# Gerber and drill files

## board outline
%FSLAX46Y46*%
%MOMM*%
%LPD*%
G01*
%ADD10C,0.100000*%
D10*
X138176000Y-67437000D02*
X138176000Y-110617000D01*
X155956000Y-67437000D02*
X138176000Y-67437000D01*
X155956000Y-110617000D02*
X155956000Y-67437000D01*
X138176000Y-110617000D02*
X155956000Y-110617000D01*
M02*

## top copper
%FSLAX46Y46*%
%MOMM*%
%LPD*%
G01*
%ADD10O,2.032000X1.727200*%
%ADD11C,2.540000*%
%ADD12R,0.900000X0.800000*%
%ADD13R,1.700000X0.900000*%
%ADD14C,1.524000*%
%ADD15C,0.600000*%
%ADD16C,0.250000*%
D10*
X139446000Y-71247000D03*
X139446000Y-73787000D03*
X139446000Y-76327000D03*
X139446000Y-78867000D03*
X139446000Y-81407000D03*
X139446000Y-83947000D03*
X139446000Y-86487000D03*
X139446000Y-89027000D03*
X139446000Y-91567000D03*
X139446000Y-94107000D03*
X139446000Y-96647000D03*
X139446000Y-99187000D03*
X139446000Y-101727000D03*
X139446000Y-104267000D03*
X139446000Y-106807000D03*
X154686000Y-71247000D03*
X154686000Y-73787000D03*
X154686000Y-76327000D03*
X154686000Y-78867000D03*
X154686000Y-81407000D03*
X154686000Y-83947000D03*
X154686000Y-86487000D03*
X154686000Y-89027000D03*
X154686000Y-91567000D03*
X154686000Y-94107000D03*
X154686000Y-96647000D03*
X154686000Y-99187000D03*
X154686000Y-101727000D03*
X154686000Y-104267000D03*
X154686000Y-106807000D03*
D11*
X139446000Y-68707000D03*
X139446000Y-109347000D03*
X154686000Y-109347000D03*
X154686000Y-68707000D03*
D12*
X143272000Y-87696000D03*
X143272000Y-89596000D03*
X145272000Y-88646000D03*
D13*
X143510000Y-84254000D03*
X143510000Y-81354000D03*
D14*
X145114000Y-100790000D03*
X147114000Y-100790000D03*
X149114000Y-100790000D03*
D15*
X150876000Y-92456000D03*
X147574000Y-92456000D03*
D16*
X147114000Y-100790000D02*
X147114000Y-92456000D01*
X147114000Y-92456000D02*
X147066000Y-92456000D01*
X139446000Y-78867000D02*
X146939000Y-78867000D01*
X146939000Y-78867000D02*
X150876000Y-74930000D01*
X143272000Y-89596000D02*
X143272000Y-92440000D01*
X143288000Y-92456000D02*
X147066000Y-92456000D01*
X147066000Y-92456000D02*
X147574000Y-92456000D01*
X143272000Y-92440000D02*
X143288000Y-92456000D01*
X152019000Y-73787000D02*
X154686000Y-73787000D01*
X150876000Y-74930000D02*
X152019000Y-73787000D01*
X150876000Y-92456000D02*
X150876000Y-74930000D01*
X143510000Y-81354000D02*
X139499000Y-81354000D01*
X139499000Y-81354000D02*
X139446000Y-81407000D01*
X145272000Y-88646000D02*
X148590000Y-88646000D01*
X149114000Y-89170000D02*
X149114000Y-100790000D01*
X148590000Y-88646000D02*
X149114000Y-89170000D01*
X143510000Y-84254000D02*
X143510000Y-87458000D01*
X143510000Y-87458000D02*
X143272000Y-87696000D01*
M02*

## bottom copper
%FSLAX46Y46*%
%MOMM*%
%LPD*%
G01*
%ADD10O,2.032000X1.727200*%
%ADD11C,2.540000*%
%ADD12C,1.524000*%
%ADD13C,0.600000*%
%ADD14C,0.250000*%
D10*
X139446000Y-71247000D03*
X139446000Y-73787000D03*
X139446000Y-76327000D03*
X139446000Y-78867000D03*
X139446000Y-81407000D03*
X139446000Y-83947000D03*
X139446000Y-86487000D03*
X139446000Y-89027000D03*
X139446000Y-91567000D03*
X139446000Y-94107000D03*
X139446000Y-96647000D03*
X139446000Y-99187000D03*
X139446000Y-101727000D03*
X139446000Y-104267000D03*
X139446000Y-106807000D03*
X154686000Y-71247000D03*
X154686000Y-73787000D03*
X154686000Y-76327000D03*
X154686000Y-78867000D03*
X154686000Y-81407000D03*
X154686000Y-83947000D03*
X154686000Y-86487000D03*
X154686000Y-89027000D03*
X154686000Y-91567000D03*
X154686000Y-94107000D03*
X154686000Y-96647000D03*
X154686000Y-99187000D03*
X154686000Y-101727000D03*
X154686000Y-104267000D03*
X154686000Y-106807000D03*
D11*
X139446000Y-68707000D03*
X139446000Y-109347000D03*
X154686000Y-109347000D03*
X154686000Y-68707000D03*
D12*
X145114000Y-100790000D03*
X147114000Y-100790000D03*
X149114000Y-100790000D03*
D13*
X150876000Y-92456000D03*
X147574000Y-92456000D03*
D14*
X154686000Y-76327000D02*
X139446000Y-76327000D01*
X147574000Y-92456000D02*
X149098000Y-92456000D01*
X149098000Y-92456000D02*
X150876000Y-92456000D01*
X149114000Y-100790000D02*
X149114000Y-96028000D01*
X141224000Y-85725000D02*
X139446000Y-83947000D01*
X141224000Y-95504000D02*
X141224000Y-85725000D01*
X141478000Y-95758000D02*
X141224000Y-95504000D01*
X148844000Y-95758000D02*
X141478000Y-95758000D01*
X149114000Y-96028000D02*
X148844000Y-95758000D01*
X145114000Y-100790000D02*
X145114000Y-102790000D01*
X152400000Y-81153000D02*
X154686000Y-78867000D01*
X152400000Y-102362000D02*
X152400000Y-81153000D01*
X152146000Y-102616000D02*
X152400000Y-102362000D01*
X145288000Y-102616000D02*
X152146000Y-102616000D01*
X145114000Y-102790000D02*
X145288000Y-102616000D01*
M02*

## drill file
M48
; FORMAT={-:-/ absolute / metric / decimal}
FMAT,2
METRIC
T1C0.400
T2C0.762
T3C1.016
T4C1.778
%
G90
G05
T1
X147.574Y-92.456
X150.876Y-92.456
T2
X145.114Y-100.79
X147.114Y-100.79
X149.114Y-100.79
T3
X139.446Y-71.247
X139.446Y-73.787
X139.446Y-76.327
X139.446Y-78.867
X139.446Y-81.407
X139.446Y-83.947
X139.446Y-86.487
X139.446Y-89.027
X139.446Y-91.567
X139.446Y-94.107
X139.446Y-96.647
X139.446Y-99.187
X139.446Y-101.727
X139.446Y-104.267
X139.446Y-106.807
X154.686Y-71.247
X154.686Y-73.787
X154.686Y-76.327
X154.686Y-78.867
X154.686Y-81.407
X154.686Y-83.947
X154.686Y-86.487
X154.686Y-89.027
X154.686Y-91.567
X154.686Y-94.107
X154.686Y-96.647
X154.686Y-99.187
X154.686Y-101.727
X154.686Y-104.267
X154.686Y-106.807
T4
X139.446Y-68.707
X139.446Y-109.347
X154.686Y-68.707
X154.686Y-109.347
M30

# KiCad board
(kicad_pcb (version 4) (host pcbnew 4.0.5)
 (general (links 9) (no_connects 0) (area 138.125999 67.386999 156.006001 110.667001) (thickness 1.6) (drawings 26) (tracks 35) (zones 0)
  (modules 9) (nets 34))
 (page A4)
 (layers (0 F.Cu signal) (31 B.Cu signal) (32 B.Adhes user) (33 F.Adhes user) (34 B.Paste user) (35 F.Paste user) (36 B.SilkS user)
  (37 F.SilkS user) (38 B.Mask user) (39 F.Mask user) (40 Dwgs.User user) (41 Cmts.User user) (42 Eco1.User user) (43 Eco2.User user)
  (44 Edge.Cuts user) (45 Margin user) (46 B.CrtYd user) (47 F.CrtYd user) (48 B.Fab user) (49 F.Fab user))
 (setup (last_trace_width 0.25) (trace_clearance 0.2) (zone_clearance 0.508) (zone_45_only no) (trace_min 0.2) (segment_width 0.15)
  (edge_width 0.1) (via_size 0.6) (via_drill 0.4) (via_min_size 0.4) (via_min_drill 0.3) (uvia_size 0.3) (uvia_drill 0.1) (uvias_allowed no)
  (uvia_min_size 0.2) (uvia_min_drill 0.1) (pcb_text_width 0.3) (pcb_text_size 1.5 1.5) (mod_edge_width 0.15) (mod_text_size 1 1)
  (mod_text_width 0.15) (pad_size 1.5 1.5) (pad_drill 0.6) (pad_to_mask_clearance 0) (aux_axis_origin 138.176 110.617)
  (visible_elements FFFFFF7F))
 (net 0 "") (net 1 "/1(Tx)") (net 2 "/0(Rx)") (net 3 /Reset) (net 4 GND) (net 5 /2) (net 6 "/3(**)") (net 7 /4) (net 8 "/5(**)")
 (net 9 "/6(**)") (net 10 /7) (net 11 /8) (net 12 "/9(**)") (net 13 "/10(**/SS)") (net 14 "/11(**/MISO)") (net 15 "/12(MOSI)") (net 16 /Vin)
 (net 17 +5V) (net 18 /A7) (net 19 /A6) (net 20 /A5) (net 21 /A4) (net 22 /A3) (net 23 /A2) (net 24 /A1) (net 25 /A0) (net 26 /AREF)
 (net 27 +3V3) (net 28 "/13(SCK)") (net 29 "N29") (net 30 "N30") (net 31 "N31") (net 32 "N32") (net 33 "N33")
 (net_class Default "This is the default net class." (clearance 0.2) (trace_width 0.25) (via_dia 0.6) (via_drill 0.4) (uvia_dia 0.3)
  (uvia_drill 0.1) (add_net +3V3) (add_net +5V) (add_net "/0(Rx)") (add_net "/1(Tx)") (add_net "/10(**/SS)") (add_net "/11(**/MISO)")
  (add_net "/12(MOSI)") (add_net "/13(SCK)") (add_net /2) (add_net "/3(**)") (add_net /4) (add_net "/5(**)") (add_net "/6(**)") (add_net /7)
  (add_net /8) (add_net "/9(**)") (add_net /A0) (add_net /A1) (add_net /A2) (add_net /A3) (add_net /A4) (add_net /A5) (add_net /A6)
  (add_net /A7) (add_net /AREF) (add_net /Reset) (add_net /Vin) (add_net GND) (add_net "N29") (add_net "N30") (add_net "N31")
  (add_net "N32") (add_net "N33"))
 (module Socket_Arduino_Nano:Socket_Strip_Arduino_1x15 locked (layer F.Cu) (at 139.446 71.247 270)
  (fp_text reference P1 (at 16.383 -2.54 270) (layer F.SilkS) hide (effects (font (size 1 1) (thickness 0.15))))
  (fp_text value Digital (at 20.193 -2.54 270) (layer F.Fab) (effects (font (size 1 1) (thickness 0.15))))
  (pad 1 thru_hole oval (at 0 0 270) (size 1.7272 2.032) (drill 1.016) (layers *.Cu *.Mask F.SilkS) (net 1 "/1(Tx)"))
  (pad 2 thru_hole oval (at 2.54 0 270) (size 1.7272 2.032) (drill 1.016) (layers *.Cu *.Mask F.SilkS) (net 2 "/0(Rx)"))
  (pad 3 thru_hole oval (at 5.08 0 270) (size 1.7272 2.032) (drill 1.016) (layers *.Cu *.Mask F.SilkS) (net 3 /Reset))
  (pad 4 thru_hole oval (at 7.62 0 270) (size 1.7272 2.032) (drill 1.016) (layers *.Cu *.Mask F.SilkS) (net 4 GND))
  (pad 5 thru_hole oval (at 10.16 0 270) (size 1.7272 2.032) (drill 1.016) (layers *.Cu *.Mask F.SilkS) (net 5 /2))
  (pad 6 thru_hole oval (at 12.7 0 270) (size 1.7272 2.032) (drill 1.016) (layers *.Cu *.Mask F.SilkS) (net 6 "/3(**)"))
  (pad 7 thru_hole oval (at 15.24 0 270) (size 1.7272 2.032) (drill 1.016) (layers *.Cu *.Mask F.SilkS) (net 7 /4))
  (pad 8 thru_hole oval (at 17.78 0 270) (size 1.7272 2.032) (drill 1.016) (layers *.Cu *.Mask F.SilkS) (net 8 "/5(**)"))
  (pad 9 thru_hole oval (at 20.32 0 270) (size 1.7272 2.032) (drill 1.016) (layers *.Cu *.Mask F.SilkS) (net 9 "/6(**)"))
  (pad 10 thru_hole oval (at 22.86 0 270) (size 1.7272 2.032) (drill 1.016) (layers *.Cu *.Mask F.SilkS) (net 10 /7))
  (pad 11 thru_hole oval (at 25.4 0 270) (size 1.7272 2.032) (drill 1.016) (layers *.Cu *.Mask F.SilkS) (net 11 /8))
  (pad 12 thru_hole oval (at 27.94 0 270) (size 1.7272 2.032) (drill 1.016) (layers *.Cu *.Mask F.SilkS) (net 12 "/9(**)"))
  (pad 13 thru_hole oval (at 30.48 0 270) (size 1.7272 2.032) (drill 1.016) (layers *.Cu *.Mask F.SilkS) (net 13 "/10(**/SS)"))
  (pad 14 thru_hole oval (at 33.02 0 270) (size 1.7272 2.032) (drill 1.016) (layers *.Cu *.Mask F.SilkS) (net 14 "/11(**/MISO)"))
  (pad 15 thru_hole oval (at 35.56 0 270) (size 1.7272 2.032) (drill 1.016) (layers *.Cu *.Mask F.SilkS) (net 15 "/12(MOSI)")))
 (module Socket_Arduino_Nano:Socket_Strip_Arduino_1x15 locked (layer F.Cu) (at 154.686 71.247 270)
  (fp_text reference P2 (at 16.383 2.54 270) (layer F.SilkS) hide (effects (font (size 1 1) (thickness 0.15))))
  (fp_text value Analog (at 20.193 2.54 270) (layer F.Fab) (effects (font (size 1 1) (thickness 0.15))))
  (pad 1 thru_hole oval (at 0 0 270) (size 1.7272 2.032) (drill 1.016) (layers *.Cu *.Mask F.SilkS) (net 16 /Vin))
  (pad 2 thru_hole oval (at 2.54 0 270) (size 1.7272 2.032) (drill 1.016) (layers *.Cu *.Mask F.SilkS) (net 4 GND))
  (pad 3 thru_hole oval (at 5.08 0 270) (size 1.7272 2.032) (drill 1.016) (layers *.Cu *.Mask F.SilkS) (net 3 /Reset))
  (pad 4 thru_hole oval (at 7.62 0 270) (size 1.7272 2.032) (drill 1.016) (layers *.Cu *.Mask F.SilkS) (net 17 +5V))
  (pad 5 thru_hole oval (at 10.16 0 270) (size 1.7272 2.032) (drill 1.016) (layers *.Cu *.Mask F.SilkS) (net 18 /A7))
  (pad 6 thru_hole oval (at 12.7 0 270) (size 1.7272 2.032) (drill 1.016) (layers *.Cu *.Mask F.SilkS) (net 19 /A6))
  (pad 7 thru_hole oval (at 15.24 0 270) (size 1.7272 2.032) (drill 1.016) (layers *.Cu *.Mask F.SilkS) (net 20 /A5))
  (pad 8 thru_hole oval (at 17.78 0 270) (size 1.7272 2.032) (drill 1.016) (layers *.Cu *.Mask F.SilkS) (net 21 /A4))
  (pad 9 thru_hole oval (at 20.32 0 270) (size 1.7272 2.032) (drill 1.016) (layers *.Cu *.Mask F.SilkS) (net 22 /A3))
  (pad 10 thru_hole oval (at 22.86 0 270) (size 1.7272 2.032) (drill 1.016) (layers *.Cu *.Mask F.SilkS) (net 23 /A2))
  (pad 11 thru_hole oval (at 25.4 0 270) (size 1.7272 2.032) (drill 1.016) (layers *.Cu *.Mask F.SilkS) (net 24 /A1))
  (pad 12 thru_hole oval (at 27.94 0 270) (size 1.7272 2.032) (drill 1.016) (layers *.Cu *.Mask F.SilkS) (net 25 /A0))
  (pad 13 thru_hole oval (at 30.48 0 270) (size 1.7272 2.032) (drill 1.016) (layers *.Cu *.Mask F.SilkS) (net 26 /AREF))
  (pad 14 thru_hole oval (at 33.02 0 270) (size 1.7272 2.032) (drill 1.016) (layers *.Cu *.Mask F.SilkS) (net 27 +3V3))
  (pad 15 thru_hole oval (at 35.56 0 270) (size 1.7272 2.032) (drill 1.016) (layers *.Cu *.Mask F.SilkS) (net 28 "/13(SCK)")))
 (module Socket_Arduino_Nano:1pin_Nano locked (layer F.Cu) (at 139.446 68.707)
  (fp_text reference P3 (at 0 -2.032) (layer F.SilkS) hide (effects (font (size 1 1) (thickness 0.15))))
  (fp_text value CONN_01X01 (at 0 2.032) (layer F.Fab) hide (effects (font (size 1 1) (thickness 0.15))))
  (pad 1 thru_hole circle (at 0 0) (size 2.54 2.54) (drill 1.778) (layers *.Cu *.Mask F.SilkS) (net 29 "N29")))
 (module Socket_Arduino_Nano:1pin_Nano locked (layer F.Cu) (at 139.446 109.347)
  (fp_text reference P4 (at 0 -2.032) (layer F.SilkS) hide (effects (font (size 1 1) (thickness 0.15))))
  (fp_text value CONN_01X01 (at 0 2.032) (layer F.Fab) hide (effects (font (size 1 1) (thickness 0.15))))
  (pad 1 thru_hole circle (at 0 0) (size 2.54 2.54) (drill 1.778) (layers *.Cu *.Mask F.SilkS) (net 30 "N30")))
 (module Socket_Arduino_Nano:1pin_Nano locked (layer F.Cu) (at 154.686 109.347)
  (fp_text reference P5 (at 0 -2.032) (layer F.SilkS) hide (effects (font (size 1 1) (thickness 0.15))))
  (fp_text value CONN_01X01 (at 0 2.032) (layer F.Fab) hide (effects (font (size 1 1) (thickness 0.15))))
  (pad 1 thru_hole circle (at 0 0) (size 2.54 2.54) (drill 1.778) (layers *.Cu *.Mask F.SilkS) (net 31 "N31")))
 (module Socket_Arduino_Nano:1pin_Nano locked (layer F.Cu) (at 154.686 68.707)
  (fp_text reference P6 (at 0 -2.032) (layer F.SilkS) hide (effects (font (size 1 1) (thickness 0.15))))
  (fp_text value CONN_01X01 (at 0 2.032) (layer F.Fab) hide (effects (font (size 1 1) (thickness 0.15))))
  (pad 1 thru_hole circle (at 0 0) (size 2.54 2.54) (drill 1.778) (layers *.Cu *.Mask F.SilkS) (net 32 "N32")))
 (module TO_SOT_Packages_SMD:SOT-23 (layer F.Cu) (at 144.272 88.646)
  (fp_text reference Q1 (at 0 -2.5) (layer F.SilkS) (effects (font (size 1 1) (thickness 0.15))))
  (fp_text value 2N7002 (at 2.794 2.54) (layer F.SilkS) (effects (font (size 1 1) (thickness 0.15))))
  (pad 1 smd rect (at -1 -0.95) (size 0.9 0.8) (layers F.Cu F.Paste F.Mask) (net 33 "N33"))
  (pad 2 smd rect (at -1 0.95) (size 0.9 0.8) (layers F.Cu F.Paste F.Mask) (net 4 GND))
  (pad 3 smd rect (at 1 0) (size 0.9 0.8) (layers F.Cu F.Paste F.Mask) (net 6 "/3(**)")))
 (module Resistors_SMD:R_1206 (layer F.Cu) (at 143.51 82.804 90)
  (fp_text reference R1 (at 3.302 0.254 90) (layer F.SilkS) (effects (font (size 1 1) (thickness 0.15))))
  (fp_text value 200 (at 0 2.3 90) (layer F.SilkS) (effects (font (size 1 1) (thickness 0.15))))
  (pad 1 smd rect (at -1.45 0 90) (size 0.9 1.7) (layers F.Cu F.Paste F.Mask) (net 33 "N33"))
  (pad 2 smd rect (at 1.45 0 90) (size 0.9 1.7) (layers F.Cu F.Paste F.Mask) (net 5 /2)))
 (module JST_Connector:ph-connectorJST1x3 (layer F.Cu) (at 150.114 97.79)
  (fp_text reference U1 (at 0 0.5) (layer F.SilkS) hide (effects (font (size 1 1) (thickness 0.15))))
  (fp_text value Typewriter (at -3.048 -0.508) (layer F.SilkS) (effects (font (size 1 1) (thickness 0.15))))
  (pad 1 thru_hole circle (at -5 3) (size 1.524 1.524) (drill 0.762) (layers *.Cu *.Mask) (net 17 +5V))
  (pad 2 thru_hole circle (at -3 3) (size 1.524 1.524) (drill 0.762) (layers *.Cu *.Mask) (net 4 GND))
  (pad 3 thru_hole circle (at -1 3) (size 1.524 1.524) (drill 0.762) (layers *.Cu *.Mask) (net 6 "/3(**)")))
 (gr_line (start 138.176 67.437) (end 138.176 110.617) (angle 90) (layer Edge.Cuts) (width 0.1))
 (gr_line (start 155.956 67.437) (end 138.176 67.437) (angle 90) (layer Edge.Cuts) (width 0.1))
 (gr_line (start 155.956 110.617) (end 155.956 67.437) (angle 90) (layer Edge.Cuts) (width 0.1))
 (gr_line (start 138.176 110.617) (end 155.956 110.617) (angle 90) (layer Edge.Cuts) (width 0.1))
 (segment (start 154.686 76.327) (end 139.446 76.327) (width 0.25) (layer B.Cu) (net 3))
 (segment (start 147.114 100.79) (end 147.114 92.456) (width 0.25) (layer F.Cu) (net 4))
 (segment (start 147.114 92.456) (end 147.066 92.456) (width 0.25) (layer F.Cu) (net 4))
 (segment (start 139.446 78.867) (end 146.939 78.867) (width 0.25) (layer F.Cu) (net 4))
 (segment (start 146.939 78.867) (end 150.876 74.93) (width 0.25) (layer F.Cu) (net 4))
 (segment (start 143.272 89.596) (end 143.272 92.44) (width 0.25) (layer F.Cu) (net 4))
 (via (at 150.876 92.456) (size 0.6) (drill 0.4) (layers F.Cu B.Cu) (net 4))
 (segment (start 147.574 92.456) (end 149.098 92.456) (width 0.25) (layer B.Cu) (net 4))
 (segment (start 149.098 92.456) (end 150.876 92.456) (width 0.25) (layer B.Cu) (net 4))
 (via (at 147.574 92.456) (size 0.6) (drill 0.4) (layers F.Cu B.Cu) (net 4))
 (segment (start 143.288 92.456) (end 147.066 92.456) (width 0.25) (layer F.Cu) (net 4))
 (segment (start 147.066 92.456) (end 147.574 92.456) (width 0.25) (layer F.Cu) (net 4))
 (segment (start 143.272 92.44) (end 143.288 92.456) (width 0.25) (layer F.Cu) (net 4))
 (segment (start 152.019 73.787) (end 154.686 73.787) (width 0.25) (layer F.Cu) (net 4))
 (segment (start 150.876 74.93) (end 152.019 73.787) (width 0.25) (layer F.Cu) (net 4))
 (segment (start 150.876 92.456) (end 150.876 74.93) (width 0.25) (layer F.Cu) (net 4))
 (segment (start 143.51 81.354) (end 139.499 81.354) (width 0.25) (layer F.Cu) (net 5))
 (segment (start 139.499 81.354) (end 139.446 81.407) (width 0.25) (layer F.Cu) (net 5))
 (segment (start 145.272 88.646) (end 148.59 88.646) (width 0.25) (layer F.Cu) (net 6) (status 400000))
 (segment (start 149.114 89.17) (end 149.114 100.79) (width 0.25) (layer F.Cu) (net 6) (status 800000))
 (segment (start 148.59 88.646) (end 149.114 89.17) (width 0.25) (layer F.Cu) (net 6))
 (segment (start 149.114 100.79) (end 149.114 96.028) (width 0.25) (layer B.Cu) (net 6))
 (segment (start 141.224 85.725) (end 139.446 83.947) (width 0.25) (layer B.Cu) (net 6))
 (segment (start 141.224 95.504) (end 141.224 85.725) (width 0.25) (layer B.Cu) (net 6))
 (segment (start 141.478 95.758) (end 141.224 95.504) (width 0.25) (layer B.Cu) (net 6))
 (segment (start 148.844 95.758) (end 141.478 95.758) (width 0.25) (layer B.Cu) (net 6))
 (segment (start 149.114 96.028) (end 148.844 95.758) (width 0.25) (layer B.Cu) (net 6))
 (segment (start 145.114 100.79) (end 145.114 102.79) (width 0.25) (layer B.Cu) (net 17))
 (segment (start 152.4 81.153) (end 154.686 78.867) (width 0.25) (layer B.Cu) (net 17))
 (segment (start 152.4 102.362) (end 152.4 81.153) (width 0.25) (layer B.Cu) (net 17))
 (segment (start 152.146 102.616) (end 152.4 102.362) (width 0.25) (layer B.Cu) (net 17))
 (segment (start 145.288 102.616) (end 152.146 102.616) (width 0.25) (layer B.Cu) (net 17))
 (segment (start 145.114 102.79) (end 145.288 102.616) (width 0.25) (layer B.Cu) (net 17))
 (segment (start 143.51 84.254) (end 143.51 87.458) (width 0.25) (layer F.Cu) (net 33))
 (segment (start 143.51 87.458) (end 143.272 87.696) (width 0.25) (layer F.Cu) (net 33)))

